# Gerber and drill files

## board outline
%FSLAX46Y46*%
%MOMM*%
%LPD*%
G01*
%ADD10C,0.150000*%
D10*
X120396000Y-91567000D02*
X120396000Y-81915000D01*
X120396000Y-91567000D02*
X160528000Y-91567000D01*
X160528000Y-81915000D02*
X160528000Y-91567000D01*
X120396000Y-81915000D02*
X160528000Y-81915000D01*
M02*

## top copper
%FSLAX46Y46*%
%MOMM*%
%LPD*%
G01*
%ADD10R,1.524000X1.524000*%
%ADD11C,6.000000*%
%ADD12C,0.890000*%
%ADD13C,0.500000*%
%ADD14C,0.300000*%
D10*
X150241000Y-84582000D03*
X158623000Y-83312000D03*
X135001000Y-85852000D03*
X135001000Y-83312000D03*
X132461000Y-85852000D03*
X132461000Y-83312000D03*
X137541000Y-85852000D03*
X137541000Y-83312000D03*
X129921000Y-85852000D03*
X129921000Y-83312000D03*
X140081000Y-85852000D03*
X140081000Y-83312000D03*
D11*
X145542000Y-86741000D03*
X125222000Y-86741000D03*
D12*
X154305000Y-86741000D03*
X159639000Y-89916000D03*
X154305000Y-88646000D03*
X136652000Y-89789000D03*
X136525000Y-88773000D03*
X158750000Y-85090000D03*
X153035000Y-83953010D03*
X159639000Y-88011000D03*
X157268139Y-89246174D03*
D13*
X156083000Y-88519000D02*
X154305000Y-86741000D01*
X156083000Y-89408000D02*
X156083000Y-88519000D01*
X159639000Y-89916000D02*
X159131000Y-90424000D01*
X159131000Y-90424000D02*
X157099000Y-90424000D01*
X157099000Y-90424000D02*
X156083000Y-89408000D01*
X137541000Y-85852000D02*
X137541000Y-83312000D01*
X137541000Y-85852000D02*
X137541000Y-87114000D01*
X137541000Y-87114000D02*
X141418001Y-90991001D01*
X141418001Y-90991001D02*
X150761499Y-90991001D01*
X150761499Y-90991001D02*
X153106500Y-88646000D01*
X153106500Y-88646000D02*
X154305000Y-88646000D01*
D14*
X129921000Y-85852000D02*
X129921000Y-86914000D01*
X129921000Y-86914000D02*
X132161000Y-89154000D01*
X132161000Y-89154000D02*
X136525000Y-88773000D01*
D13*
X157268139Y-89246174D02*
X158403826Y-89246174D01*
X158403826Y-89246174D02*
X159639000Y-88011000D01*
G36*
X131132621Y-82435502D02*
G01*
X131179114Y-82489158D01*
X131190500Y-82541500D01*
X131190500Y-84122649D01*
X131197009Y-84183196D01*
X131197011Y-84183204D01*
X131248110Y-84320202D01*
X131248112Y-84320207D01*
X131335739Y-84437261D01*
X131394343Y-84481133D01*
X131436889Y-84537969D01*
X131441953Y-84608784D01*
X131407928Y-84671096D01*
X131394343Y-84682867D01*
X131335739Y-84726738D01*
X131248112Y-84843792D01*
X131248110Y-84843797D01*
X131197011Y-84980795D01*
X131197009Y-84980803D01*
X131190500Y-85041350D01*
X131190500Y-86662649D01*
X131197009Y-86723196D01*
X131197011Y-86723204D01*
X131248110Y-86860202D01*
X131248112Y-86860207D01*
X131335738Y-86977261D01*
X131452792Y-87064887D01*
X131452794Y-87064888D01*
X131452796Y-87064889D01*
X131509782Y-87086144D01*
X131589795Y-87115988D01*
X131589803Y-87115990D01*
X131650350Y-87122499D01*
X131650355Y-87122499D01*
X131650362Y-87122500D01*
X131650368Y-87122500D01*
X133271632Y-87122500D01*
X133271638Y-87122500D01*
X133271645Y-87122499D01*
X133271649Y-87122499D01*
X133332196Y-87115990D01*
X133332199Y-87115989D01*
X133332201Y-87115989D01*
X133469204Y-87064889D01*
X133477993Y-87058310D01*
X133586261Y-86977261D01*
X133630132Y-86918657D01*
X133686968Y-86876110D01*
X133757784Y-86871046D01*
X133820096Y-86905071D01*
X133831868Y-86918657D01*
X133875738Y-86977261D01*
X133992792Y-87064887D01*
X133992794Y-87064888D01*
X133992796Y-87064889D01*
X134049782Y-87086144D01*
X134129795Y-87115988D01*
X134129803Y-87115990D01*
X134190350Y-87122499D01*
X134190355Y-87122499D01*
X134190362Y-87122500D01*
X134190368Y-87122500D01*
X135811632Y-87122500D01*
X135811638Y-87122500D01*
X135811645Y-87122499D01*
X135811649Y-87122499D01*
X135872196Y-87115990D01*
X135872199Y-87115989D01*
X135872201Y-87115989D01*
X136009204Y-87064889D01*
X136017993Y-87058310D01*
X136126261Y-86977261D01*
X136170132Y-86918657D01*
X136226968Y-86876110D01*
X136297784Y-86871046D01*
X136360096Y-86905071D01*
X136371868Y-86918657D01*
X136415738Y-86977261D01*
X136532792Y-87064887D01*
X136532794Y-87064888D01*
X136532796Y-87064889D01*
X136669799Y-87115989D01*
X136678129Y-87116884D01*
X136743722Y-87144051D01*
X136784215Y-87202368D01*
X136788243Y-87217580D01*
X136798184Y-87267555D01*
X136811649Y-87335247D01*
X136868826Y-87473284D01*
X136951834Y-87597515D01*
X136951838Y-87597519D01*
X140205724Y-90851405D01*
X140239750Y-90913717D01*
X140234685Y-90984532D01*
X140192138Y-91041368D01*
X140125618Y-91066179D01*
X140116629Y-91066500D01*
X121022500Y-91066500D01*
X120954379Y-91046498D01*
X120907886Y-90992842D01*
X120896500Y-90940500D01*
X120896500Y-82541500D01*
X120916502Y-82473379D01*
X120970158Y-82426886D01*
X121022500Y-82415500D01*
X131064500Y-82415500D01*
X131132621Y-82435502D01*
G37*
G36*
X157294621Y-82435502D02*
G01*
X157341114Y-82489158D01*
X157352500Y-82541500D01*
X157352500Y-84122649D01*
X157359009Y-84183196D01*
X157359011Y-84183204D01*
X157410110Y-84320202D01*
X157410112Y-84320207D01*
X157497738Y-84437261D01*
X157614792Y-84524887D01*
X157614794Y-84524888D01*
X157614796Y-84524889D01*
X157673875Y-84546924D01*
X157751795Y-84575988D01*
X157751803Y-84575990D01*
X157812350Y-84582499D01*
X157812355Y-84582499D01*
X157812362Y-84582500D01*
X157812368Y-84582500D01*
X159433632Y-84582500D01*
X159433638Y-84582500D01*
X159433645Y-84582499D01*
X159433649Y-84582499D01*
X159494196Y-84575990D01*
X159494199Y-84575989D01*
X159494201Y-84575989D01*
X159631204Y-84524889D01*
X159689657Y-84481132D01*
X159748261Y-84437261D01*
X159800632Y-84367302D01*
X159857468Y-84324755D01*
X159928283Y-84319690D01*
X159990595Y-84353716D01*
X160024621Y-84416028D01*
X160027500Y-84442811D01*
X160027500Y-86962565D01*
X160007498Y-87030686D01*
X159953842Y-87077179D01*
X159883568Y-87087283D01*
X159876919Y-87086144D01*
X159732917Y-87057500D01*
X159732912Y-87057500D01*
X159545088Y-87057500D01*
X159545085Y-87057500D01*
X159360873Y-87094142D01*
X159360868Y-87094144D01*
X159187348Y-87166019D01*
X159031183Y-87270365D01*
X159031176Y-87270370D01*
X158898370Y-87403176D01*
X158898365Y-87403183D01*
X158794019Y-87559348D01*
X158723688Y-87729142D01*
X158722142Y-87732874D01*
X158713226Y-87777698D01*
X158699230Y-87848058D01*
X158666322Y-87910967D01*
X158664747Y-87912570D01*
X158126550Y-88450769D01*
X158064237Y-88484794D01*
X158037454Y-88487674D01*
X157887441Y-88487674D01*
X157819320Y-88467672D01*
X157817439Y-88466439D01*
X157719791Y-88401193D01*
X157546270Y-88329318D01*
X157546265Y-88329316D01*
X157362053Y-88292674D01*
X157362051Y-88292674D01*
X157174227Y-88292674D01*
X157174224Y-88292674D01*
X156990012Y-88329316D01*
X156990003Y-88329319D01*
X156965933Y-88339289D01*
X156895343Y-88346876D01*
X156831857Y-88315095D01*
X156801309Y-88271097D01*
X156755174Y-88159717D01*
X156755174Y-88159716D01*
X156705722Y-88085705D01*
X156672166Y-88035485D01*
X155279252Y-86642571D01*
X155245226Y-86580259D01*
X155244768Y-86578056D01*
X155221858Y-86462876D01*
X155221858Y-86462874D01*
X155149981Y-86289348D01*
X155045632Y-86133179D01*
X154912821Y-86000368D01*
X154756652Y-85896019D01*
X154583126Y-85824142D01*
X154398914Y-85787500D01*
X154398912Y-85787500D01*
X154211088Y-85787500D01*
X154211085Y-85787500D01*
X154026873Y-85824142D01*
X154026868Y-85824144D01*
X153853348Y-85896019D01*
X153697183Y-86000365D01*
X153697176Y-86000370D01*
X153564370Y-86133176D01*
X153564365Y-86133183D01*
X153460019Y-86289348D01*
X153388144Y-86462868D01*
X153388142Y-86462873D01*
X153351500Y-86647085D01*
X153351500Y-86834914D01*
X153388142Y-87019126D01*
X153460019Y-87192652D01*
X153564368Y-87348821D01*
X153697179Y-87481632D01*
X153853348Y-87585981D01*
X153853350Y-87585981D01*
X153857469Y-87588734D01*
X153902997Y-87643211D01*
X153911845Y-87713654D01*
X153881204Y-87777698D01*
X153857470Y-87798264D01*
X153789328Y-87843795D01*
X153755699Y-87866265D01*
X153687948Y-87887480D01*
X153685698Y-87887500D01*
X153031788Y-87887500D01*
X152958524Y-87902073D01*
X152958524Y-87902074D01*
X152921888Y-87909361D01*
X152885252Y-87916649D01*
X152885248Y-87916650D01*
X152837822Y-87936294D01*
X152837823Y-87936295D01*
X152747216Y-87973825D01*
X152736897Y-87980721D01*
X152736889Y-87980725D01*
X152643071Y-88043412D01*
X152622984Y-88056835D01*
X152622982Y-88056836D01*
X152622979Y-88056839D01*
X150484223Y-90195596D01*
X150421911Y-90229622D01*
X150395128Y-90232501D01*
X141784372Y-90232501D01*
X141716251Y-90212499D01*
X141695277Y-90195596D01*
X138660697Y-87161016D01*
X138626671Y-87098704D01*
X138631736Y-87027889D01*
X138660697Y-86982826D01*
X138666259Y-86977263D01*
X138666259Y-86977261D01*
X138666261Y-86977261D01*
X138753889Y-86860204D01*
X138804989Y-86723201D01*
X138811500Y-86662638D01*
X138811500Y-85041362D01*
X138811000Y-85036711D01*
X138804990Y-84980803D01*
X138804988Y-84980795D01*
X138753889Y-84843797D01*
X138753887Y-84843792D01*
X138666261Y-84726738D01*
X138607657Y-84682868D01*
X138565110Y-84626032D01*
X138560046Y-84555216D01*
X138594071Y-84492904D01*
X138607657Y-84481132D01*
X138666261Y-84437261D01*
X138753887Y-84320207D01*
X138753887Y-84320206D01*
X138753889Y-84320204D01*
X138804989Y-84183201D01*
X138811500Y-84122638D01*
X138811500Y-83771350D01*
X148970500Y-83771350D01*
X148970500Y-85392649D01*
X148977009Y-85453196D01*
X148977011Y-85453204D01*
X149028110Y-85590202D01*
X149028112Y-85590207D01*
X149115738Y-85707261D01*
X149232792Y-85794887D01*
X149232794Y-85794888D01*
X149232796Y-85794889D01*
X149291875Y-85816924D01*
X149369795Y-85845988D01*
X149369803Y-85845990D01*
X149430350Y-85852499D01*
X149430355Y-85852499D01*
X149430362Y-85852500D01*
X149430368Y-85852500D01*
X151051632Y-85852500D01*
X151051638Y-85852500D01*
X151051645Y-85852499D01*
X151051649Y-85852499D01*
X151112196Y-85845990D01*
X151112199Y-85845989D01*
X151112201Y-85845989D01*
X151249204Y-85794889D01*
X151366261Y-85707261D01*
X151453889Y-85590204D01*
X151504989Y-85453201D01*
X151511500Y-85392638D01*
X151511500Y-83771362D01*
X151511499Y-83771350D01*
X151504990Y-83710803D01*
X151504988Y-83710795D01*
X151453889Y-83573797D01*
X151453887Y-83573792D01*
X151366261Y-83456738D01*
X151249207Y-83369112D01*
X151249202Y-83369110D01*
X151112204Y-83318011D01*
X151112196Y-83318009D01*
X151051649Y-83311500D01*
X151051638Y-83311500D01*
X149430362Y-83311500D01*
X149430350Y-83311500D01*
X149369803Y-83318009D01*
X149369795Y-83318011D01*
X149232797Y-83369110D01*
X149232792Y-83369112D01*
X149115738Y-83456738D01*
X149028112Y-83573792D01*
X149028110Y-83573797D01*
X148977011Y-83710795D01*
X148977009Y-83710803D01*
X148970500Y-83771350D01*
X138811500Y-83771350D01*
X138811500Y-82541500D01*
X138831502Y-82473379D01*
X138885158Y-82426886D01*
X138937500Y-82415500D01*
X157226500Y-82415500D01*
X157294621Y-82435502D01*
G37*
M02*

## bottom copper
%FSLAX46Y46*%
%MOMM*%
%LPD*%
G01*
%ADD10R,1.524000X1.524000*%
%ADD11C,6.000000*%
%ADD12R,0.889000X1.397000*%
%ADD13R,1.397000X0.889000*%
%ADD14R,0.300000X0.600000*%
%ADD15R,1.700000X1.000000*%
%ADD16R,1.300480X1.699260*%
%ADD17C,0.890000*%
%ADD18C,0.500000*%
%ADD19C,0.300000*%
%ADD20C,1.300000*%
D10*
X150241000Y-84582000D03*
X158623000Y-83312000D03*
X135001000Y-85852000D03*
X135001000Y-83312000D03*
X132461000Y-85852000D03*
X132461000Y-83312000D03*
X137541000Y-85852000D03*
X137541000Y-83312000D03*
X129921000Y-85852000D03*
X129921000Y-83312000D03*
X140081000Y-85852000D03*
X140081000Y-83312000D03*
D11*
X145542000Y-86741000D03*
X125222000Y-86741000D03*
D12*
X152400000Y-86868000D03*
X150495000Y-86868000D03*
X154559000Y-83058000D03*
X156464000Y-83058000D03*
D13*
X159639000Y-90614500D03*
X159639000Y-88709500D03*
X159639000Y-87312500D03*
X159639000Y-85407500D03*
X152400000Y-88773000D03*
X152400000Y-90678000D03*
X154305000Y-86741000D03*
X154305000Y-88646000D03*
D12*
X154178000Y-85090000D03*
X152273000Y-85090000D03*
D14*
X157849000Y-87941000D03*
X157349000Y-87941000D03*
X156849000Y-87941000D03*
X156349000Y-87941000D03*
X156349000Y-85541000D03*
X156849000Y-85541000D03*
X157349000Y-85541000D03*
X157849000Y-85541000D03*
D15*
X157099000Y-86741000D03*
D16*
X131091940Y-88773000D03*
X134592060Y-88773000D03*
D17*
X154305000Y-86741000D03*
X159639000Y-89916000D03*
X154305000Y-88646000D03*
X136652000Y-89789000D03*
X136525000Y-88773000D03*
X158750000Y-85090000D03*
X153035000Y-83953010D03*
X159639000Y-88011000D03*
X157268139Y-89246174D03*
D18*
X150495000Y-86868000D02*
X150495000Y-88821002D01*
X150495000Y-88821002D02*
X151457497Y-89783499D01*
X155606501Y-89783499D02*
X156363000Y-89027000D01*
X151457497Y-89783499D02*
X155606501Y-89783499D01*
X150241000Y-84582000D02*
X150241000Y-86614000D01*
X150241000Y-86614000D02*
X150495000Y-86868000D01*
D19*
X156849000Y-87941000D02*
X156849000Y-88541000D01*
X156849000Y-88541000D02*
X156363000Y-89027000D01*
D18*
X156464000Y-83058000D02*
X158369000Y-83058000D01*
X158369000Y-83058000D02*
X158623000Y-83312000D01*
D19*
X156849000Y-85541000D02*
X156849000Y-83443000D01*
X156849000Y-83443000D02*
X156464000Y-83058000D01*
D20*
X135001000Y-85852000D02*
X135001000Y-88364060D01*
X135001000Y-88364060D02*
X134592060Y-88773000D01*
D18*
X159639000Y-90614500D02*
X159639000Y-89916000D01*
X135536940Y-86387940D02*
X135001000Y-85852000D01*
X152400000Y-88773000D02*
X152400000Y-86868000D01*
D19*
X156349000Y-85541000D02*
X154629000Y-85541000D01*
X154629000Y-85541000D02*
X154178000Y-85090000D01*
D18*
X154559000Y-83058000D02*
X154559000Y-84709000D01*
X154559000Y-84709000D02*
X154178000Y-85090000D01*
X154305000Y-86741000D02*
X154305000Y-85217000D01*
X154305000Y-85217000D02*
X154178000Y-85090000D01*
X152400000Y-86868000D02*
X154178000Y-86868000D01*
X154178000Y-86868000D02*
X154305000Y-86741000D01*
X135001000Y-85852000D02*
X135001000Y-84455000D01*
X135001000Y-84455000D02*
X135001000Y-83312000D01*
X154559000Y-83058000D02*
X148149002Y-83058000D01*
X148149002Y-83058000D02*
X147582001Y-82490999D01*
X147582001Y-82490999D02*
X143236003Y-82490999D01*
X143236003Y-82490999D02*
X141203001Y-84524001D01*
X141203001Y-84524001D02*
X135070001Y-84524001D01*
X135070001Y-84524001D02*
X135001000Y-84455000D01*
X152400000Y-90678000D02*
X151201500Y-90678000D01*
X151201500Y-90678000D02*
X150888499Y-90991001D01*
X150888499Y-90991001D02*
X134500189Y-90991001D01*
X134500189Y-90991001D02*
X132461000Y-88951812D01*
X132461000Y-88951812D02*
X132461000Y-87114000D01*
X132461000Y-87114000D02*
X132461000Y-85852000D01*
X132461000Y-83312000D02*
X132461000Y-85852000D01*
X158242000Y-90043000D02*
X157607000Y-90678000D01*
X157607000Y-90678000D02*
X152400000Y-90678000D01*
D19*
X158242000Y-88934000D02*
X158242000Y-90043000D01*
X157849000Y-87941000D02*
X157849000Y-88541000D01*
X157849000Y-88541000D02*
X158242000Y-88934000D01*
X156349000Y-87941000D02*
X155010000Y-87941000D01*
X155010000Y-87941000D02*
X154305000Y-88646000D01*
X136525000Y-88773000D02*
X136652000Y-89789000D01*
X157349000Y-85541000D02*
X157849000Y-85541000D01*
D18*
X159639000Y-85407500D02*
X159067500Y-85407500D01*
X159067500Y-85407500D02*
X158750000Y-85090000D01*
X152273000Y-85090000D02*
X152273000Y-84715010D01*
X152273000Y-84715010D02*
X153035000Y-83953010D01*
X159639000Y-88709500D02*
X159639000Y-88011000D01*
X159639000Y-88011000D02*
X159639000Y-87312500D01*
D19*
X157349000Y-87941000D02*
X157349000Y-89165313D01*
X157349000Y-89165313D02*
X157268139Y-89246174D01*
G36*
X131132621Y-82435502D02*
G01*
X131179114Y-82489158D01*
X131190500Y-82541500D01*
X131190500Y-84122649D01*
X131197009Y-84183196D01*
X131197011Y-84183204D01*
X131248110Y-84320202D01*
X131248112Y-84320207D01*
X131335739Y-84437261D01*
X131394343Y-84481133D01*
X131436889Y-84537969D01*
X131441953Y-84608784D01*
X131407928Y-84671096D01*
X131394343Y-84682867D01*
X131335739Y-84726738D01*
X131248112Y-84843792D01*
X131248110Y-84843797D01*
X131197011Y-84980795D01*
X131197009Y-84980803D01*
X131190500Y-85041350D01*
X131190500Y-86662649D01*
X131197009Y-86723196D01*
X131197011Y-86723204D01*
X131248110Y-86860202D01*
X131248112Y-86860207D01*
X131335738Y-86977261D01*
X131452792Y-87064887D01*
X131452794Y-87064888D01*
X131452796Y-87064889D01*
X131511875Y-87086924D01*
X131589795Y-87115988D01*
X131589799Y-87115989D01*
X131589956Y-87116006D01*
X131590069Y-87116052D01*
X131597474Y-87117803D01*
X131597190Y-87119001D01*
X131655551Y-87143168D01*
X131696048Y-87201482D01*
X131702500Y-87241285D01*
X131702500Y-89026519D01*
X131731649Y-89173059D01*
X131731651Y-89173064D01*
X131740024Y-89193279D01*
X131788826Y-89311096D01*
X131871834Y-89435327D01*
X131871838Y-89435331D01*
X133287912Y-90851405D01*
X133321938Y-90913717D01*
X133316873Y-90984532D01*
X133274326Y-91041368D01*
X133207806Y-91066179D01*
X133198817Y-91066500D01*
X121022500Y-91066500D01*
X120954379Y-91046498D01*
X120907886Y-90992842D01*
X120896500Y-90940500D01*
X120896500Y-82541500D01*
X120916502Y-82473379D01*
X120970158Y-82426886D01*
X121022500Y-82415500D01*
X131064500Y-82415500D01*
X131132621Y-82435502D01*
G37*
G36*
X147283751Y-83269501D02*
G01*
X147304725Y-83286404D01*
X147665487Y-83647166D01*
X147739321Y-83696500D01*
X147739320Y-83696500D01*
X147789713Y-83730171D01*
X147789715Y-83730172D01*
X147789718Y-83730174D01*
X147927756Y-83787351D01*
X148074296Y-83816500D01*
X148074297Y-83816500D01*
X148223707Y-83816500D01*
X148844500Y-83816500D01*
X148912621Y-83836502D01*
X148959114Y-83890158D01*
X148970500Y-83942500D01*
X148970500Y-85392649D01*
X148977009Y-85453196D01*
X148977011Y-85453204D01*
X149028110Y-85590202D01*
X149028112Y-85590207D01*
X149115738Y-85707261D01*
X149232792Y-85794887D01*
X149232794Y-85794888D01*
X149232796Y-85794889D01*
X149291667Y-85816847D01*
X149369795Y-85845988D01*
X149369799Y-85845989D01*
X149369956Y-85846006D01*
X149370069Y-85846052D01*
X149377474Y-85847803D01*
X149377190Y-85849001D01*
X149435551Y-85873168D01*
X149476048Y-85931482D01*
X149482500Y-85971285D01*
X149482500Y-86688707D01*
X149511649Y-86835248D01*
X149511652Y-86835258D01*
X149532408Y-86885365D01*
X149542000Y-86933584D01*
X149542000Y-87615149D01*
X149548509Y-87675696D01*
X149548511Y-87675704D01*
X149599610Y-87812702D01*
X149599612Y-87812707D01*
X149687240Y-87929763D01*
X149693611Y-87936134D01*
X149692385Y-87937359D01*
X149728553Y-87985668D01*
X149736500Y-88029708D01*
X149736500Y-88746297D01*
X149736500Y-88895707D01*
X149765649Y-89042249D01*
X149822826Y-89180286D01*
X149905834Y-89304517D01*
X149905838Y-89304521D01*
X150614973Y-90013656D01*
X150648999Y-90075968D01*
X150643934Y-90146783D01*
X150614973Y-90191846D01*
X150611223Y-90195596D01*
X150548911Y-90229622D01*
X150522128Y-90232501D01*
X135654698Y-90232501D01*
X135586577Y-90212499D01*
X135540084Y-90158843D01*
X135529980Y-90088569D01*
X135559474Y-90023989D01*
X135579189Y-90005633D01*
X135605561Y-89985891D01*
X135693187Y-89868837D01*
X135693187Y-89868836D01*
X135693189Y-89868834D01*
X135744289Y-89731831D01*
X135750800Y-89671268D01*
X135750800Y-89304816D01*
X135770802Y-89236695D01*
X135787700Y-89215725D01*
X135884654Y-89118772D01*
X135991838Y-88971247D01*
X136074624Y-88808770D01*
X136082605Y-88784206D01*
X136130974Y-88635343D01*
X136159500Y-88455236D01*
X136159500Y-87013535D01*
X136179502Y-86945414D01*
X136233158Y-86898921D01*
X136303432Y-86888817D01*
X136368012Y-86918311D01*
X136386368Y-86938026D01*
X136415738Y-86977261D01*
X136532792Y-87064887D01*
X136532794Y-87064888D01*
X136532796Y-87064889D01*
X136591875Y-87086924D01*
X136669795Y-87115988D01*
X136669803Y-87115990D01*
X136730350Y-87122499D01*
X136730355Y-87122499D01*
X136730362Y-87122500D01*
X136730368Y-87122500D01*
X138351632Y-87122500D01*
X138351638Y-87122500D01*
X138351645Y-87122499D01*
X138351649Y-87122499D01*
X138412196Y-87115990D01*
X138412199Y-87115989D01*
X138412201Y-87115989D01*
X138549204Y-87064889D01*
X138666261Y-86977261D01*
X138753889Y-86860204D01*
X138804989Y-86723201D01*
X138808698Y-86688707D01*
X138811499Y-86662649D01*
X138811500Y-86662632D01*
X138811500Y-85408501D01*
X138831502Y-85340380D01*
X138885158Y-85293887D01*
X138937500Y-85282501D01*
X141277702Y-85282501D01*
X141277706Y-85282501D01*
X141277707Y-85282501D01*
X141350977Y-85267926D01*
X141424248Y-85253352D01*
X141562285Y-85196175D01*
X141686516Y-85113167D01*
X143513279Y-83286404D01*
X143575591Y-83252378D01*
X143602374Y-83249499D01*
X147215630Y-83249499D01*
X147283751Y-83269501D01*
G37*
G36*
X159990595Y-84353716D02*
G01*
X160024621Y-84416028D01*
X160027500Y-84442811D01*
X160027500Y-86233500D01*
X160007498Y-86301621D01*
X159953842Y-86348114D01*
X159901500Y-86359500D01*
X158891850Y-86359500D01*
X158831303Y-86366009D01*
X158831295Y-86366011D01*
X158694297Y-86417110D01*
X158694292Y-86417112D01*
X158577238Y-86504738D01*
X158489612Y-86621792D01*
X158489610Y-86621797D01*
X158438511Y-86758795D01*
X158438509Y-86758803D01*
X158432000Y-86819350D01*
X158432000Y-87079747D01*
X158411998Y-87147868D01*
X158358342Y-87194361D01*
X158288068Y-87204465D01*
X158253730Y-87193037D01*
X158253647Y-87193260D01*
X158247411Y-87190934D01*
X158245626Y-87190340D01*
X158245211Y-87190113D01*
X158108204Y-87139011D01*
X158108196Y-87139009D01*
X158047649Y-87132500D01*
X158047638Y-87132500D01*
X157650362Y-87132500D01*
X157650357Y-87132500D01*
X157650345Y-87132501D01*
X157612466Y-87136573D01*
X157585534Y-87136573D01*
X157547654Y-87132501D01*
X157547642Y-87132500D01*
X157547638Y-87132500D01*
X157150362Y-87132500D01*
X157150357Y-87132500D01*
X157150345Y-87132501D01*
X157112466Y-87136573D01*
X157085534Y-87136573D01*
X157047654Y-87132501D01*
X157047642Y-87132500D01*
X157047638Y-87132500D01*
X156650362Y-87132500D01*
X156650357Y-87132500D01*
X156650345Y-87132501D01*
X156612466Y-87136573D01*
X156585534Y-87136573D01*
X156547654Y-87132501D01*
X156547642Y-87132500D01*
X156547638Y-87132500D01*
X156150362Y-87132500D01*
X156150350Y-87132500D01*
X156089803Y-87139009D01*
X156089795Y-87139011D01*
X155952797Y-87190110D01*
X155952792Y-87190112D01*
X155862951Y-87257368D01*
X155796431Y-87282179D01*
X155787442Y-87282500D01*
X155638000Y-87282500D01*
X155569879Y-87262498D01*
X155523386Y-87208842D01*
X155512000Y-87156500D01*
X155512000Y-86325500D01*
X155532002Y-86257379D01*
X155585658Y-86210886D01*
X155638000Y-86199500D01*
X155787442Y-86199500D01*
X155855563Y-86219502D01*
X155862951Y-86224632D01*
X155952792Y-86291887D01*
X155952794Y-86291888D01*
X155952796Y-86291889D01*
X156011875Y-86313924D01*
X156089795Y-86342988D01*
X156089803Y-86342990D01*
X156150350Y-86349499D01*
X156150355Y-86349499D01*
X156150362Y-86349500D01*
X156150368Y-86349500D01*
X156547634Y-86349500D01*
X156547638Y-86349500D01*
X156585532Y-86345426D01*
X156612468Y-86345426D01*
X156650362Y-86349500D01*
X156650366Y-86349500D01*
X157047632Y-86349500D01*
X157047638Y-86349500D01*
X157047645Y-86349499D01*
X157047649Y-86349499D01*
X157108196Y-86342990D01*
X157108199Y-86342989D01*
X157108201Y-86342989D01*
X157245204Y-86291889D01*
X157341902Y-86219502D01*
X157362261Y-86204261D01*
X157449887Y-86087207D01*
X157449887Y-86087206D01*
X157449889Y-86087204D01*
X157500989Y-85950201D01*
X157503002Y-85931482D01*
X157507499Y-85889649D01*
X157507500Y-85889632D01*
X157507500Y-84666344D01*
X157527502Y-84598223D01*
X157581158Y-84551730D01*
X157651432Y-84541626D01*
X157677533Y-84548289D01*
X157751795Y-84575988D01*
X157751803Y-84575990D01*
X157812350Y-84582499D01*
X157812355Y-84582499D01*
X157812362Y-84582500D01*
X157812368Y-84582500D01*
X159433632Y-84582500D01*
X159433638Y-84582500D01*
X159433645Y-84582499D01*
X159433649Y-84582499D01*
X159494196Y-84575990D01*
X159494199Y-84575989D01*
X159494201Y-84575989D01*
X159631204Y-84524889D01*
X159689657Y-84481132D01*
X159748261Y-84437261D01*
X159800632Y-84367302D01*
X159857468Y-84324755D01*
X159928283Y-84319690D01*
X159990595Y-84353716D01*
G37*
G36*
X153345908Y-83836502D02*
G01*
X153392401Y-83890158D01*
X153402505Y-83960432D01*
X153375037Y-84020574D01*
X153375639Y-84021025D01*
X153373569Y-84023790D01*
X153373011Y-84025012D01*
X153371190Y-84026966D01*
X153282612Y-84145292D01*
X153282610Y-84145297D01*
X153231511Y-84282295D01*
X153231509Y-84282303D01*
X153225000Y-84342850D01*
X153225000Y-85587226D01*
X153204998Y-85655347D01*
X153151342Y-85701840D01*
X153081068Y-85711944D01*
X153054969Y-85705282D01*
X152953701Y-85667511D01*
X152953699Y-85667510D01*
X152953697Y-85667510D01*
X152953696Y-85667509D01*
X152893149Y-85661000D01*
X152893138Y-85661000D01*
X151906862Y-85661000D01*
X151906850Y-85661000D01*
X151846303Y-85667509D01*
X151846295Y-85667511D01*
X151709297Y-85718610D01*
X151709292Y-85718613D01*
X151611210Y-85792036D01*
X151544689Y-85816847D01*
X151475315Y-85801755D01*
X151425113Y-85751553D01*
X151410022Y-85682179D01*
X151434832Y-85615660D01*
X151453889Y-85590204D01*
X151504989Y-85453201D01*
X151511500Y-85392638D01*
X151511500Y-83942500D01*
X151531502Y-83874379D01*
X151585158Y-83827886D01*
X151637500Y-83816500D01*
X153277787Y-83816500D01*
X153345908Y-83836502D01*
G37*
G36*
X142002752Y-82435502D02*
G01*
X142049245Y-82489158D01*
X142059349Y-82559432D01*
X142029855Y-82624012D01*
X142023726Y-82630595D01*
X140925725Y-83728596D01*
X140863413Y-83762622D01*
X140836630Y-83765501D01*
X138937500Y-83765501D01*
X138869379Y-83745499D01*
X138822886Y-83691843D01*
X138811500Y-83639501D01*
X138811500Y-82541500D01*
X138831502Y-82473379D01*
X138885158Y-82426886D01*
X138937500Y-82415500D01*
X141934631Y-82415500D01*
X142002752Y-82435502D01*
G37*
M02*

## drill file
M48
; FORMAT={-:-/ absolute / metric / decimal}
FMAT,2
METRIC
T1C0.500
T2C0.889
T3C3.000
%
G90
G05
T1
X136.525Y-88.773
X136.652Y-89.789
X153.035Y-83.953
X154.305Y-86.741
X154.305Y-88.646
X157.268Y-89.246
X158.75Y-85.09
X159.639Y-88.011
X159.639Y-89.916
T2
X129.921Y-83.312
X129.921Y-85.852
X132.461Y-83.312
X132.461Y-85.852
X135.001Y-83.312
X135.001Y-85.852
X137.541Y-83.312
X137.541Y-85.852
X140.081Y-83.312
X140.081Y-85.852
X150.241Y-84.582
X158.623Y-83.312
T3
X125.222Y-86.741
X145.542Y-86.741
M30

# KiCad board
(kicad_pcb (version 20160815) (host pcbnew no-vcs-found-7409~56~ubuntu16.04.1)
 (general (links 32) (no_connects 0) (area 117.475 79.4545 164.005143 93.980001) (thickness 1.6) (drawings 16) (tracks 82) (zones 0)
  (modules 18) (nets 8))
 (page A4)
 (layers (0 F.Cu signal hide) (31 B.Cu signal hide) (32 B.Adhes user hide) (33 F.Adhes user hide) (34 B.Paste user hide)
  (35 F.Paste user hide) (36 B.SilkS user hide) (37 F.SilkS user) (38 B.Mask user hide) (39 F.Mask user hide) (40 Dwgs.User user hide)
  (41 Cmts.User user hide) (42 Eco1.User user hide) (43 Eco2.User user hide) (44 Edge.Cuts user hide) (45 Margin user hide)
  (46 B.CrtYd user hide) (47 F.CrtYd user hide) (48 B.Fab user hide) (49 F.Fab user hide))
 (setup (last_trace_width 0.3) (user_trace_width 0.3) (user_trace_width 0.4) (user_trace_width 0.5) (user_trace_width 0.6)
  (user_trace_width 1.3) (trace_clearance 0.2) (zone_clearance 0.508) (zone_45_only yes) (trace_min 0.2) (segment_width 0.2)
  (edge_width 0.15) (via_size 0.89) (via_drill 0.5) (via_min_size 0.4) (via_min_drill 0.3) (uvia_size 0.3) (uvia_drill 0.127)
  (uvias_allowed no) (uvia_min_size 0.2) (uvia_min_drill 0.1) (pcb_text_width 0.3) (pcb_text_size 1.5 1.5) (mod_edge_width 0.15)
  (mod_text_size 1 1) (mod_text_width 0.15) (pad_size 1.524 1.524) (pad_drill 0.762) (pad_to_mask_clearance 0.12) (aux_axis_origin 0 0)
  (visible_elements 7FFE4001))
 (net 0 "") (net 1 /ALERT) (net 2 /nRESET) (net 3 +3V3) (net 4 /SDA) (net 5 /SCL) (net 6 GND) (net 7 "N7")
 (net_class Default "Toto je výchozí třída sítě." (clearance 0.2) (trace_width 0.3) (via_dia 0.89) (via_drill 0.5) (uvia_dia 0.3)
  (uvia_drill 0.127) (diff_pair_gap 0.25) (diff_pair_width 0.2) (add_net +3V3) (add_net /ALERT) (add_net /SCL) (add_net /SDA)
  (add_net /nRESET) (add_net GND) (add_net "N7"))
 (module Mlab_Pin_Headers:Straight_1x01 (layer F.Cu) (at 150.241 84.582)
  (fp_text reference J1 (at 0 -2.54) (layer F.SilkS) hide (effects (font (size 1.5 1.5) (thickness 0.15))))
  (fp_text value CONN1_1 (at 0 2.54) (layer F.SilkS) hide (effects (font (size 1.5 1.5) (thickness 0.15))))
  (pad 1 thru_hole rect (at 0 0) (size 1.524 1.524) (drill 0.889) (layers *.Cu *.Mask F.SilkS) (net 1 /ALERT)))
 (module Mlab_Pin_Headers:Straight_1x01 (layer F.Cu) (at 158.623 83.312)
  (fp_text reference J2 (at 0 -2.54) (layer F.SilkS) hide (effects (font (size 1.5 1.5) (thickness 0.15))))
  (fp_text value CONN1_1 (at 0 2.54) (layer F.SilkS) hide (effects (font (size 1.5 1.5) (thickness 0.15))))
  (pad 1 thru_hole rect (at 0 0) (size 1.524 1.524) (drill 0.889) (layers *.Cu *.Mask F.SilkS) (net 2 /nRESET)))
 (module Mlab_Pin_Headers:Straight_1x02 (layer F.Cu) (at 135.001 84.582)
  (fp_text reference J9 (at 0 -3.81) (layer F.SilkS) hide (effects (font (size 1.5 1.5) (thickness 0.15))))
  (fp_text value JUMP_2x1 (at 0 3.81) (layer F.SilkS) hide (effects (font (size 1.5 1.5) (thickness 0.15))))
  (pad 2 thru_hole rect (at 0 1.27) (size 1.524 1.524) (drill 0.889) (layers *.Cu *.Mask F.SilkS) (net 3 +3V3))
  (pad 1 thru_hole rect (at 0 -1.27) (size 1.524 1.524) (drill 0.889) (layers *.Cu *.Mask F.SilkS) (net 3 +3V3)))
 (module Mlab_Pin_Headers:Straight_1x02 (layer F.Cu) (at 132.461 84.582)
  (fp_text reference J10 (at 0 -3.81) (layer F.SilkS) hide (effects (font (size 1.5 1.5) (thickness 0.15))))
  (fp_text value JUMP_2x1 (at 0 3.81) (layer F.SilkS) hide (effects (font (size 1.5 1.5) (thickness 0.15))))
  (pad 2 thru_hole rect (at 0 1.27) (size 1.524 1.524) (drill 0.889) (layers *.Cu *.Mask F.SilkS) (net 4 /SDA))
  (pad 1 thru_hole rect (at 0 -1.27) (size 1.524 1.524) (drill 0.889) (layers *.Cu *.Mask F.SilkS) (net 4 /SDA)))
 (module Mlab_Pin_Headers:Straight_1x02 (layer F.Cu) (at 137.541 84.582)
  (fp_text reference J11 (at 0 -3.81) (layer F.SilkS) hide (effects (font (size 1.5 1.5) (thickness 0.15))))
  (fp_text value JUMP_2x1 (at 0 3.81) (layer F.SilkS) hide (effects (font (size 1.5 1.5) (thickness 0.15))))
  (pad 2 thru_hole rect (at 0 1.27) (size 1.524 1.524) (drill 0.889) (layers *.Cu *.Mask F.SilkS) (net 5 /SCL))
  (pad 1 thru_hole rect (at 0 -1.27) (size 1.524 1.524) (drill 0.889) (layers *.Cu *.Mask F.SilkS) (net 5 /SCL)))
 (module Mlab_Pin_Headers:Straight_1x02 (layer F.Cu) (at 129.921 84.582)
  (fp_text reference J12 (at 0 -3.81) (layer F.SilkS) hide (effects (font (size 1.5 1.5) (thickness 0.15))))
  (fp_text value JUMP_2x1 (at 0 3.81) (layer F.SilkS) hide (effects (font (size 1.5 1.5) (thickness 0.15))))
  (pad 2 thru_hole rect (at 0 1.27) (size 1.524 1.524) (drill 0.889) (layers *.Cu *.Mask F.SilkS) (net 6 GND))
  (pad 1 thru_hole rect (at 0 -1.27) (size 1.524 1.524) (drill 0.889) (layers *.Cu *.Mask F.SilkS) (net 6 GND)))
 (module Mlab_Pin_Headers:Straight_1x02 (layer F.Cu) (at 140.081 84.582)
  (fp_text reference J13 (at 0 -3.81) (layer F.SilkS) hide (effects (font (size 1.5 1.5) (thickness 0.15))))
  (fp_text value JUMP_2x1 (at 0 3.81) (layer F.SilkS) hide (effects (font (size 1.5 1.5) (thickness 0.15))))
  (pad 2 thru_hole rect (at 0 1.27) (size 1.524 1.524) (drill 0.889) (layers *.Cu *.Mask F.SilkS) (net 6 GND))
  (pad 1 thru_hole rect (at 0 -1.27) (size 1.524 1.524) (drill 0.889) (layers *.Cu *.Mask F.SilkS) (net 6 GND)))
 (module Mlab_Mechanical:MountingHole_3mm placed (layer F.Cu) (at 145.542 86.741)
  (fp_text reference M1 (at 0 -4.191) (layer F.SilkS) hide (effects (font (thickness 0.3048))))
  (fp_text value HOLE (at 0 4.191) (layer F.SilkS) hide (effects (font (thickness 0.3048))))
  (pad 1 thru_hole circle (at 0 0) (size 6 6) (drill 3) (layers *.Cu *.Adhes *.Mask) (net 6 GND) (clearance 1) (zone_connect 2)))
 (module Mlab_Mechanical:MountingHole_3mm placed (layer F.Cu) (at 125.222 86.741)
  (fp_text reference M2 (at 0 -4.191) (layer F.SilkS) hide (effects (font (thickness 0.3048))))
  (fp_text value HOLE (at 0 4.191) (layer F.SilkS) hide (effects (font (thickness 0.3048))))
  (pad 1 thru_hole circle (at 0 0) (size 6 6) (drill 3) (layers *.Cu *.Adhes *.Mask) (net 6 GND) (clearance 1) (zone_connect 2)))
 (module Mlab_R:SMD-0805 (layer B.Cu) (at 151.4475 86.868 180)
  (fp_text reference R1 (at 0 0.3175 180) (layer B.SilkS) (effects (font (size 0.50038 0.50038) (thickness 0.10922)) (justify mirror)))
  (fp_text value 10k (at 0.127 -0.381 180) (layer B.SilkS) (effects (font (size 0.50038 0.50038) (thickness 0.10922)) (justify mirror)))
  (pad 1 smd rect (at -0.9525 0 180) (size 0.889 1.397) (layers B.Cu B.Paste B.Mask) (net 3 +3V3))
  (pad 2 smd rect (at 0.9525 0 180) (size 0.889 1.397) (layers B.Cu B.Paste B.Mask) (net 1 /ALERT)))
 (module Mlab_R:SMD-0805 (layer B.Cu) (at 155.5115 83.058)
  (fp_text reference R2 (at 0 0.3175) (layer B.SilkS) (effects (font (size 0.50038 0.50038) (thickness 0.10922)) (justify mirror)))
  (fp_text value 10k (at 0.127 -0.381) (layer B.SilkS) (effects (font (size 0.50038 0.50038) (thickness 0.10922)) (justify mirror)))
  (pad 1 smd rect (at -0.9525 0) (size 0.889 1.397) (layers B.Cu B.Paste B.Mask) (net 3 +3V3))
  (pad 2 smd rect (at 0.9525 0) (size 0.889 1.397) (layers B.Cu B.Paste B.Mask) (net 2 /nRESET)))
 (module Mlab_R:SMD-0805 (layer B.Cu) (at 159.639 89.662 90)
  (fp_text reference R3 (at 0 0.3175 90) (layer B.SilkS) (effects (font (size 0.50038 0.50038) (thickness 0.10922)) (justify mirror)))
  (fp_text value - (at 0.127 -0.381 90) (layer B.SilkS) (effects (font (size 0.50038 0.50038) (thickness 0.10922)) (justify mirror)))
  (pad 1 smd rect (at -0.9525 0 90) (size 0.889 1.397) (layers B.Cu B.Paste B.Mask) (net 3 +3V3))
  (pad 2 smd rect (at 0.9525 0 90) (size 0.889 1.397) (layers B.Cu B.Paste B.Mask) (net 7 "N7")))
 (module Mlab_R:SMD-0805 (layer B.Cu) (at 159.639 86.36 90)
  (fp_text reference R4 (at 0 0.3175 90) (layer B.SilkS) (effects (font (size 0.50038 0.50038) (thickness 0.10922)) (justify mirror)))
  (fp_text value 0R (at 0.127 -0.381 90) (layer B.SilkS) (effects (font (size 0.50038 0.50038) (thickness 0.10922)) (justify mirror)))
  (pad 1 smd rect (at -0.9525 0 90) (size 0.889 1.397) (layers B.Cu B.Paste B.Mask) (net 7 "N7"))
  (pad 2 smd rect (at 0.9525 0 90) (size 0.889 1.397) (layers B.Cu B.Paste B.Mask) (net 6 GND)))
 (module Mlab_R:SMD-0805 (layer B.Cu) (at 152.4 89.7255 270)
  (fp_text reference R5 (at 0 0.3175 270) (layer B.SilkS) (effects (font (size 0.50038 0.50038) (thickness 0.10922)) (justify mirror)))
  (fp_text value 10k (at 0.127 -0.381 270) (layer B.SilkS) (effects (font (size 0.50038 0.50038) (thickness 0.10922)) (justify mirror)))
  (pad 1 smd rect (at -0.9525 0 270) (size 0.889 1.397) (layers B.Cu B.Paste B.Mask) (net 3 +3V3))
  (pad 2 smd rect (at 0.9525 0 270) (size 0.889 1.397) (layers B.Cu B.Paste B.Mask) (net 4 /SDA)))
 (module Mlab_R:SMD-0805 (layer B.Cu) (at 154.305 87.6935 270)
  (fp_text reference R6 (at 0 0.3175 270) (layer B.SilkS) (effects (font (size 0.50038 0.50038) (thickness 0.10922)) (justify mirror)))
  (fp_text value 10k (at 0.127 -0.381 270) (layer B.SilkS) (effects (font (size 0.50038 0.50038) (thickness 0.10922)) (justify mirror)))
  (pad 1 smd rect (at -0.9525 0 270) (size 0.889 1.397) (layers B.Cu B.Paste B.Mask) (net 3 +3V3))
  (pad 2 smd rect (at 0.9525 0 270) (size 0.889 1.397) (layers B.Cu B.Paste B.Mask) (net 5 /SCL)))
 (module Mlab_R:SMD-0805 (layer B.Cu) (at 153.2255 85.09 180)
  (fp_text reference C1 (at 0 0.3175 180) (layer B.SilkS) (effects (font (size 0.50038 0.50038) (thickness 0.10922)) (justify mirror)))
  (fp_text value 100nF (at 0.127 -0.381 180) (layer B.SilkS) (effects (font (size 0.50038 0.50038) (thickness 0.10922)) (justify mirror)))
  (pad 1 smd rect (at -0.9525 0 180) (size 0.889 1.397) (layers B.Cu B.Paste B.Mask) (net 3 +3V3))
  (pad 2 smd rect (at 0.9525 0 180) (size 0.889 1.397) (layers B.Cu B.Paste B.Mask) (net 6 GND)))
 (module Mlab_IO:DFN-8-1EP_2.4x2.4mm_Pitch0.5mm (layer B.Cu) (at 157.099 86.741 90)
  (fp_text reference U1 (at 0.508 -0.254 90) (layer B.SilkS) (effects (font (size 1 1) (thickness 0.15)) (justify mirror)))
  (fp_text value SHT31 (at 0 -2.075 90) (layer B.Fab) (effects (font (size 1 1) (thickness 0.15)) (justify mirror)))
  (pad 1 smd rect (at -1.2 0.75 90) (size 0.6 0.3) (layers B.Cu B.Paste B.Mask) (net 4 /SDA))
  (pad 2 smd rect (at -1.2 0.25 90) (size 0.6 0.3) (layers B.Cu B.Paste B.Mask) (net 7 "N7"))
  (pad 3 smd rect (at -1.2 -0.25 90) (size 0.6 0.3) (layers B.Cu B.Paste B.Mask) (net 1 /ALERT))
  (pad 4 smd rect (at -1.2 -0.75 90) (size 0.6 0.3) (layers B.Cu B.Paste B.Mask) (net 5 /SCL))
  (pad 5 smd rect (at 1.2 -0.75 90) (size 0.6 0.3) (layers B.Cu B.Paste B.Mask) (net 3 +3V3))
  (pad 6 smd rect (at 1.2 -0.25 90) (size 0.6 0.3) (layers B.Cu B.Paste B.Mask) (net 2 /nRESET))
  (pad 7 smd rect (at 1.2 0.25 90) (size 0.6 0.3) (layers B.Cu B.Paste B.Mask) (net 6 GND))
  (pad 8 smd rect (at 1.2 0.75 90) (size 0.6 0.3) (layers B.Cu B.Paste B.Mask) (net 6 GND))
  (pad 9 smd rect (at 0 0 90) (size 1 1.7) (layers B.Cu B.Paste B.Mask) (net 6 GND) (solder_paste_margin_ratio -0.2)))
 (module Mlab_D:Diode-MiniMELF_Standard (layer B.Cu) (at 132.842 88.773)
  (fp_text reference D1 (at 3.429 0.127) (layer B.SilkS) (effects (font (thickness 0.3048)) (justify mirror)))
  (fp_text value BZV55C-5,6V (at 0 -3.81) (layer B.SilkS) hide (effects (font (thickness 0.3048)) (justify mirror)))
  (pad 1 smd rect (at -1.75006 0) (size 1.30048 1.69926) (layers B.Cu B.Paste B.Mask) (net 6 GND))
  (pad 2 smd rect (at 1.75006 0) (size 1.30048 1.69926) (layers B.Cu B.Paste B.Mask) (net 3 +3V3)))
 (gr_line (start 120.396 91.567) (end 120.396 81.915) (angle 90) (layer Edge.Cuts) (width 0.15))
 (gr_line (start 120.396 91.567) (end 160.528 91.567) (angle 90) (layer Edge.Cuts) (width 0.15))
 (gr_line (start 160.528 81.915) (end 160.528 91.567) (angle 90) (layer Edge.Cuts) (width 0.15))
 (gr_line (start 120.396 81.915) (end 160.528 81.915) (angle 90) (layer Edge.Cuts) (width 0.15))
 (segment (start 150.495 86.868) (end 150.495 88.821002) (width 0.5) (layer B.Cu) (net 1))
 (segment (start 150.495 88.821002) (end 151.457497 89.783499) (width 0.5) (layer B.Cu) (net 1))
 (segment (start 155.606501 89.783499) (end 156.363 89.027) (width 0.5) (layer B.Cu) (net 1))
 (segment (start 151.457497 89.783499) (end 155.606501 89.783499) (width 0.5) (layer B.Cu) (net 1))
 (segment (start 150.241 84.582) (end 150.241 86.614) (width 0.5) (layer B.Cu) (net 1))
 (segment (start 150.241 86.614) (end 150.495 86.868) (width 0.5) (layer B.Cu) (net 1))
 (segment (start 156.849 87.941) (end 156.849 88.541) (width 0.3) (layer B.Cu) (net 1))
 (segment (start 156.849 88.541) (end 156.363 89.027) (width 0.3) (layer B.Cu) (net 1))
 (segment (start 156.464 83.058) (end 158.369 83.058) (width 0.5) (layer B.Cu) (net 2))
 (segment (start 158.369 83.058) (end 158.623 83.312) (width 0.5) (layer B.Cu) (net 2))
 (segment (start 156.849 85.541) (end 156.849 83.443) (width 0.3) (layer B.Cu) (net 2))
 (segment (start 156.849 83.443) (end 156.464 83.058) (width 0.3) (layer B.Cu) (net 2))
 (segment (start 135.001 85.852) (end 135.001 88.36406) (width 1.3) (layer B.Cu) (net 3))
 (segment (start 135.001 88.36406) (end 134.59206 88.773) (width 1.3) (layer B.Cu) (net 3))
 (segment (start 156.083 88.519) (end 154.305 86.741) (width 0.5) (layer F.Cu) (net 3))
 (segment (start 156.083 89.408) (end 156.083 88.519) (width 0.5) (layer F.Cu) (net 3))
 (segment (start 159.639 89.916) (end 159.131 90.424) (width 0.5) (layer F.Cu) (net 3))
 (segment (start 159.131 90.424) (end 157.099 90.424) (width 0.5) (layer F.Cu) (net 3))
 (segment (start 157.099 90.424) (end 156.083 89.408) (width 0.5) (layer F.Cu) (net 3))
 (via (at 154.305 86.741) (size 0.89) (drill 0.5) (layers F.Cu B.Cu) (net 3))
 (segment (start 159.639 90.6145) (end 159.639 89.916) (width 0.5) (layer B.Cu) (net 3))
 (via (at 159.639 89.916) (size 0.89) (drill 0.5) (layers F.Cu B.Cu) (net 3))
 (segment (start 135.53694 86.38794) (end 135.001 85.852) (width 0.5) (layer B.Cu) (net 3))
 (segment (start 152.4 88.773) (end 152.4 86.868) (width 0.5) (layer B.Cu) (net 3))
 (segment (start 156.349 85.541) (end 154.629 85.541) (width 0.3) (layer B.Cu) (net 3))
 (segment (start 154.629 85.541) (end 154.178 85.09) (width 0.3) (layer B.Cu) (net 3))
 (segment (start 154.559 83.058) (end 154.559 84.709) (width 0.5) (layer B.Cu) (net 3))
 (segment (start 154.559 84.709) (end 154.178 85.09) (width 0.5) (layer B.Cu) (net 3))
 (segment (start 154.305 86.741) (end 154.305 85.217) (width 0.5) (layer B.Cu) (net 3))
 (segment (start 154.305 85.217) (end 154.178 85.09) (width 0.5) (layer B.Cu) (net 3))
 (segment (start 152.4 86.868) (end 154.178 86.868) (width 0.5) (layer B.Cu) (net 3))
 (segment (start 154.178 86.868) (end 154.305 86.741) (width 0.5) (layer B.Cu) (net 3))
 (segment (start 135.001 85.852) (end 135.001 84.455) (width 0.5) (layer B.Cu) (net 3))
 (segment (start 135.001 84.455) (end 135.001 83.312) (width 0.5) (layer B.Cu) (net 3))
 (segment (start 154.559 83.058) (end 148.149002 83.058) (width 0.5) (layer B.Cu) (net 3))
 (segment (start 148.149002 83.058) (end 147.582001 82.490999) (width 0.5) (layer B.Cu) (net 3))
 (segment (start 147.582001 82.490999) (end 143.236003 82.490999) (width 0.5) (layer B.Cu) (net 3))
 (segment (start 143.236003 82.490999) (end 141.203001 84.524001) (width 0.5) (layer B.Cu) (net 3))
 (segment (start 141.203001 84.524001) (end 135.070001 84.524001) (width 0.5) (layer B.Cu) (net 3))
 (segment (start 135.070001 84.524001) (end 135.001 84.455) (width 0.5) (layer B.Cu) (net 3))
 (segment (start 152.4 90.678) (end 151.2015 90.678) (width 0.5) (layer B.Cu) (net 4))
 (segment (start 151.2015 90.678) (end 150.888499 90.991001) (width 0.5) (layer B.Cu) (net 4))
 (segment (start 150.888499 90.991001) (end 134.500189 90.991001) (width 0.5) (layer B.Cu) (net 4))
 (segment (start 134.500189 90.991001) (end 132.461 88.951812) (width 0.5) (layer B.Cu) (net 4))
 (segment (start 132.461 88.951812) (end 132.461 87.114) (width 0.5) (layer B.Cu) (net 4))
 (segment (start 132.461 87.114) (end 132.461 85.852) (width 0.5) (layer B.Cu) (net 4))
 (segment (start 132.461 83.312) (end 132.461 85.852) (width 0.5) (layer B.Cu) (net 4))
 (segment (start 158.242 90.043) (end 157.607 90.678) (width 0.5) (layer B.Cu) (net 4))
 (segment (start 157.607 90.678) (end 152.4 90.678) (width 0.5) (layer B.Cu) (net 4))
 (segment (start 158.242 88.934) (end 158.242 90.043) (width 0.3) (layer B.Cu) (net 4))
 (segment (start 157.849 87.941) (end 157.849 88.541) (width 0.3) (layer B.Cu) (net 4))
 (segment (start 157.849 88.541) (end 158.242 88.934) (width 0.3) (layer B.Cu) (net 4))
 (segment (start 137.541 85.852) (end 137.541 83.312) (width 0.5) (layer F.Cu) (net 5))
 (segment (start 137.541 85.852) (end 137.541 87.114) (width 0.5) (layer F.Cu) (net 5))
 (segment (start 137.541 87.114) (end 141.418001 90.991001) (width 0.5) (layer F.Cu) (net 5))
 (segment (start 141.418001 90.991001) (end 150.761499 90.991001) (width 0.5) (layer F.Cu) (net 5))
 (segment (start 150.761499 90.991001) (end 153.1065 88.646) (width 0.5) (layer F.Cu) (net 5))
 (segment (start 153.1065 88.646) (end 154.305 88.646) (width 0.5) (layer F.Cu) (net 5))
 (via (at 154.305 88.646) (size 0.89) (drill 0.5) (layers F.Cu B.Cu) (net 5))
 (segment (start 156.349 87.941) (end 155.01 87.941) (width 0.3) (layer B.Cu) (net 5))
 (segment (start 155.01 87.941) (end 154.305 88.646) (width 0.3) (layer B.Cu) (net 5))
 (segment (start 136.525 88.773) (end 136.652 89.789) (width 0.3) (layer B.Cu) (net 6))
 (via (at 136.652 89.789) (size 0.89) (drill 0.5) (layers F.Cu B.Cu) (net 6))
 (segment (start 129.921 85.852) (end 129.921 86.914) (width 0.3) (layer F.Cu) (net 6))
 (segment (start 129.921 86.914) (end 132.161 89.154) (width 0.3) (layer F.Cu) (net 6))
 (segment (start 132.161 89.154) (end 136.525 88.773) (width 0.3) (layer F.Cu) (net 6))
 (via (at 136.525 88.773) (size 0.89) (drill 0.5) (layers F.Cu B.Cu) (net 6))
 (segment (start 157.349 85.541) (end 157.849 85.541) (width 0.3) (layer B.Cu) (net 6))
 (segment (start 159.639 85.4075) (end 159.0675 85.4075) (width 0.5) (layer B.Cu) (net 6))
 (segment (start 159.0675 85.4075) (end 158.75 85.09) (width 0.5) (layer B.Cu) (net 6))
 (via (at 158.75 85.09) (size 0.89) (drill 0.5) (layers F.Cu B.Cu) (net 6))
 (segment (start 152.273 85.09) (end 152.273 84.71501) (width 0.5) (layer B.Cu) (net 6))
 (segment (start 152.273 84.71501) (end 153.035 83.95301) (width 0.5) (layer B.Cu) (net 6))
 (via (at 153.035 83.95301) (size 0.89) (drill 0.5) (layers F.Cu B.Cu) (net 6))
 (segment (start 159.639 88.7095) (end 159.639 88.011) (width 0.5) (layer B.Cu) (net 7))
 (segment (start 159.639 88.011) (end 159.639 87.3125) (width 0.5) (layer B.Cu) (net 7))
 (segment (start 157.268139 89.246174) (end 158.403826 89.246174) (width 0.5) (layer F.Cu) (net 7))
 (segment (start 158.403826 89.246174) (end 159.639 88.011) (width 0.5) (layer F.Cu) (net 7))
 (via (at 159.639 88.011) (size 0.89) (drill 0.5) (layers F.Cu B.Cu) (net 7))
 (segment (start 157.349 87.941) (end 157.349 89.165313) (width 0.3) (layer B.Cu) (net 7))
 (segment (start 157.349 89.165313) (end 157.268139 89.246174) (width 0.3) (layer B.Cu) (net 7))
 (via (at 157.268139 89.246174) (size 0.89) (drill 0.5) (layers F.Cu B.Cu) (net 7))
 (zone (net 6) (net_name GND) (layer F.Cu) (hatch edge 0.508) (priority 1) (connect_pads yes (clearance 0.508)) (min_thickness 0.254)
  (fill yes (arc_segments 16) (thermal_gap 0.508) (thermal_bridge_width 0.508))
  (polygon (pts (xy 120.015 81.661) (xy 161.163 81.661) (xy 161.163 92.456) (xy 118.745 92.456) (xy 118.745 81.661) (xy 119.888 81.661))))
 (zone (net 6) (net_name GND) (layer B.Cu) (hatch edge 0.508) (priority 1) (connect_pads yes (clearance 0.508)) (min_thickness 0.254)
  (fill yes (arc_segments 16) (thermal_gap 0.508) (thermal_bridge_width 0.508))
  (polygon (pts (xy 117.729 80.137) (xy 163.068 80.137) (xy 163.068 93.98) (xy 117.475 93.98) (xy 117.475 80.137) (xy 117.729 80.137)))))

